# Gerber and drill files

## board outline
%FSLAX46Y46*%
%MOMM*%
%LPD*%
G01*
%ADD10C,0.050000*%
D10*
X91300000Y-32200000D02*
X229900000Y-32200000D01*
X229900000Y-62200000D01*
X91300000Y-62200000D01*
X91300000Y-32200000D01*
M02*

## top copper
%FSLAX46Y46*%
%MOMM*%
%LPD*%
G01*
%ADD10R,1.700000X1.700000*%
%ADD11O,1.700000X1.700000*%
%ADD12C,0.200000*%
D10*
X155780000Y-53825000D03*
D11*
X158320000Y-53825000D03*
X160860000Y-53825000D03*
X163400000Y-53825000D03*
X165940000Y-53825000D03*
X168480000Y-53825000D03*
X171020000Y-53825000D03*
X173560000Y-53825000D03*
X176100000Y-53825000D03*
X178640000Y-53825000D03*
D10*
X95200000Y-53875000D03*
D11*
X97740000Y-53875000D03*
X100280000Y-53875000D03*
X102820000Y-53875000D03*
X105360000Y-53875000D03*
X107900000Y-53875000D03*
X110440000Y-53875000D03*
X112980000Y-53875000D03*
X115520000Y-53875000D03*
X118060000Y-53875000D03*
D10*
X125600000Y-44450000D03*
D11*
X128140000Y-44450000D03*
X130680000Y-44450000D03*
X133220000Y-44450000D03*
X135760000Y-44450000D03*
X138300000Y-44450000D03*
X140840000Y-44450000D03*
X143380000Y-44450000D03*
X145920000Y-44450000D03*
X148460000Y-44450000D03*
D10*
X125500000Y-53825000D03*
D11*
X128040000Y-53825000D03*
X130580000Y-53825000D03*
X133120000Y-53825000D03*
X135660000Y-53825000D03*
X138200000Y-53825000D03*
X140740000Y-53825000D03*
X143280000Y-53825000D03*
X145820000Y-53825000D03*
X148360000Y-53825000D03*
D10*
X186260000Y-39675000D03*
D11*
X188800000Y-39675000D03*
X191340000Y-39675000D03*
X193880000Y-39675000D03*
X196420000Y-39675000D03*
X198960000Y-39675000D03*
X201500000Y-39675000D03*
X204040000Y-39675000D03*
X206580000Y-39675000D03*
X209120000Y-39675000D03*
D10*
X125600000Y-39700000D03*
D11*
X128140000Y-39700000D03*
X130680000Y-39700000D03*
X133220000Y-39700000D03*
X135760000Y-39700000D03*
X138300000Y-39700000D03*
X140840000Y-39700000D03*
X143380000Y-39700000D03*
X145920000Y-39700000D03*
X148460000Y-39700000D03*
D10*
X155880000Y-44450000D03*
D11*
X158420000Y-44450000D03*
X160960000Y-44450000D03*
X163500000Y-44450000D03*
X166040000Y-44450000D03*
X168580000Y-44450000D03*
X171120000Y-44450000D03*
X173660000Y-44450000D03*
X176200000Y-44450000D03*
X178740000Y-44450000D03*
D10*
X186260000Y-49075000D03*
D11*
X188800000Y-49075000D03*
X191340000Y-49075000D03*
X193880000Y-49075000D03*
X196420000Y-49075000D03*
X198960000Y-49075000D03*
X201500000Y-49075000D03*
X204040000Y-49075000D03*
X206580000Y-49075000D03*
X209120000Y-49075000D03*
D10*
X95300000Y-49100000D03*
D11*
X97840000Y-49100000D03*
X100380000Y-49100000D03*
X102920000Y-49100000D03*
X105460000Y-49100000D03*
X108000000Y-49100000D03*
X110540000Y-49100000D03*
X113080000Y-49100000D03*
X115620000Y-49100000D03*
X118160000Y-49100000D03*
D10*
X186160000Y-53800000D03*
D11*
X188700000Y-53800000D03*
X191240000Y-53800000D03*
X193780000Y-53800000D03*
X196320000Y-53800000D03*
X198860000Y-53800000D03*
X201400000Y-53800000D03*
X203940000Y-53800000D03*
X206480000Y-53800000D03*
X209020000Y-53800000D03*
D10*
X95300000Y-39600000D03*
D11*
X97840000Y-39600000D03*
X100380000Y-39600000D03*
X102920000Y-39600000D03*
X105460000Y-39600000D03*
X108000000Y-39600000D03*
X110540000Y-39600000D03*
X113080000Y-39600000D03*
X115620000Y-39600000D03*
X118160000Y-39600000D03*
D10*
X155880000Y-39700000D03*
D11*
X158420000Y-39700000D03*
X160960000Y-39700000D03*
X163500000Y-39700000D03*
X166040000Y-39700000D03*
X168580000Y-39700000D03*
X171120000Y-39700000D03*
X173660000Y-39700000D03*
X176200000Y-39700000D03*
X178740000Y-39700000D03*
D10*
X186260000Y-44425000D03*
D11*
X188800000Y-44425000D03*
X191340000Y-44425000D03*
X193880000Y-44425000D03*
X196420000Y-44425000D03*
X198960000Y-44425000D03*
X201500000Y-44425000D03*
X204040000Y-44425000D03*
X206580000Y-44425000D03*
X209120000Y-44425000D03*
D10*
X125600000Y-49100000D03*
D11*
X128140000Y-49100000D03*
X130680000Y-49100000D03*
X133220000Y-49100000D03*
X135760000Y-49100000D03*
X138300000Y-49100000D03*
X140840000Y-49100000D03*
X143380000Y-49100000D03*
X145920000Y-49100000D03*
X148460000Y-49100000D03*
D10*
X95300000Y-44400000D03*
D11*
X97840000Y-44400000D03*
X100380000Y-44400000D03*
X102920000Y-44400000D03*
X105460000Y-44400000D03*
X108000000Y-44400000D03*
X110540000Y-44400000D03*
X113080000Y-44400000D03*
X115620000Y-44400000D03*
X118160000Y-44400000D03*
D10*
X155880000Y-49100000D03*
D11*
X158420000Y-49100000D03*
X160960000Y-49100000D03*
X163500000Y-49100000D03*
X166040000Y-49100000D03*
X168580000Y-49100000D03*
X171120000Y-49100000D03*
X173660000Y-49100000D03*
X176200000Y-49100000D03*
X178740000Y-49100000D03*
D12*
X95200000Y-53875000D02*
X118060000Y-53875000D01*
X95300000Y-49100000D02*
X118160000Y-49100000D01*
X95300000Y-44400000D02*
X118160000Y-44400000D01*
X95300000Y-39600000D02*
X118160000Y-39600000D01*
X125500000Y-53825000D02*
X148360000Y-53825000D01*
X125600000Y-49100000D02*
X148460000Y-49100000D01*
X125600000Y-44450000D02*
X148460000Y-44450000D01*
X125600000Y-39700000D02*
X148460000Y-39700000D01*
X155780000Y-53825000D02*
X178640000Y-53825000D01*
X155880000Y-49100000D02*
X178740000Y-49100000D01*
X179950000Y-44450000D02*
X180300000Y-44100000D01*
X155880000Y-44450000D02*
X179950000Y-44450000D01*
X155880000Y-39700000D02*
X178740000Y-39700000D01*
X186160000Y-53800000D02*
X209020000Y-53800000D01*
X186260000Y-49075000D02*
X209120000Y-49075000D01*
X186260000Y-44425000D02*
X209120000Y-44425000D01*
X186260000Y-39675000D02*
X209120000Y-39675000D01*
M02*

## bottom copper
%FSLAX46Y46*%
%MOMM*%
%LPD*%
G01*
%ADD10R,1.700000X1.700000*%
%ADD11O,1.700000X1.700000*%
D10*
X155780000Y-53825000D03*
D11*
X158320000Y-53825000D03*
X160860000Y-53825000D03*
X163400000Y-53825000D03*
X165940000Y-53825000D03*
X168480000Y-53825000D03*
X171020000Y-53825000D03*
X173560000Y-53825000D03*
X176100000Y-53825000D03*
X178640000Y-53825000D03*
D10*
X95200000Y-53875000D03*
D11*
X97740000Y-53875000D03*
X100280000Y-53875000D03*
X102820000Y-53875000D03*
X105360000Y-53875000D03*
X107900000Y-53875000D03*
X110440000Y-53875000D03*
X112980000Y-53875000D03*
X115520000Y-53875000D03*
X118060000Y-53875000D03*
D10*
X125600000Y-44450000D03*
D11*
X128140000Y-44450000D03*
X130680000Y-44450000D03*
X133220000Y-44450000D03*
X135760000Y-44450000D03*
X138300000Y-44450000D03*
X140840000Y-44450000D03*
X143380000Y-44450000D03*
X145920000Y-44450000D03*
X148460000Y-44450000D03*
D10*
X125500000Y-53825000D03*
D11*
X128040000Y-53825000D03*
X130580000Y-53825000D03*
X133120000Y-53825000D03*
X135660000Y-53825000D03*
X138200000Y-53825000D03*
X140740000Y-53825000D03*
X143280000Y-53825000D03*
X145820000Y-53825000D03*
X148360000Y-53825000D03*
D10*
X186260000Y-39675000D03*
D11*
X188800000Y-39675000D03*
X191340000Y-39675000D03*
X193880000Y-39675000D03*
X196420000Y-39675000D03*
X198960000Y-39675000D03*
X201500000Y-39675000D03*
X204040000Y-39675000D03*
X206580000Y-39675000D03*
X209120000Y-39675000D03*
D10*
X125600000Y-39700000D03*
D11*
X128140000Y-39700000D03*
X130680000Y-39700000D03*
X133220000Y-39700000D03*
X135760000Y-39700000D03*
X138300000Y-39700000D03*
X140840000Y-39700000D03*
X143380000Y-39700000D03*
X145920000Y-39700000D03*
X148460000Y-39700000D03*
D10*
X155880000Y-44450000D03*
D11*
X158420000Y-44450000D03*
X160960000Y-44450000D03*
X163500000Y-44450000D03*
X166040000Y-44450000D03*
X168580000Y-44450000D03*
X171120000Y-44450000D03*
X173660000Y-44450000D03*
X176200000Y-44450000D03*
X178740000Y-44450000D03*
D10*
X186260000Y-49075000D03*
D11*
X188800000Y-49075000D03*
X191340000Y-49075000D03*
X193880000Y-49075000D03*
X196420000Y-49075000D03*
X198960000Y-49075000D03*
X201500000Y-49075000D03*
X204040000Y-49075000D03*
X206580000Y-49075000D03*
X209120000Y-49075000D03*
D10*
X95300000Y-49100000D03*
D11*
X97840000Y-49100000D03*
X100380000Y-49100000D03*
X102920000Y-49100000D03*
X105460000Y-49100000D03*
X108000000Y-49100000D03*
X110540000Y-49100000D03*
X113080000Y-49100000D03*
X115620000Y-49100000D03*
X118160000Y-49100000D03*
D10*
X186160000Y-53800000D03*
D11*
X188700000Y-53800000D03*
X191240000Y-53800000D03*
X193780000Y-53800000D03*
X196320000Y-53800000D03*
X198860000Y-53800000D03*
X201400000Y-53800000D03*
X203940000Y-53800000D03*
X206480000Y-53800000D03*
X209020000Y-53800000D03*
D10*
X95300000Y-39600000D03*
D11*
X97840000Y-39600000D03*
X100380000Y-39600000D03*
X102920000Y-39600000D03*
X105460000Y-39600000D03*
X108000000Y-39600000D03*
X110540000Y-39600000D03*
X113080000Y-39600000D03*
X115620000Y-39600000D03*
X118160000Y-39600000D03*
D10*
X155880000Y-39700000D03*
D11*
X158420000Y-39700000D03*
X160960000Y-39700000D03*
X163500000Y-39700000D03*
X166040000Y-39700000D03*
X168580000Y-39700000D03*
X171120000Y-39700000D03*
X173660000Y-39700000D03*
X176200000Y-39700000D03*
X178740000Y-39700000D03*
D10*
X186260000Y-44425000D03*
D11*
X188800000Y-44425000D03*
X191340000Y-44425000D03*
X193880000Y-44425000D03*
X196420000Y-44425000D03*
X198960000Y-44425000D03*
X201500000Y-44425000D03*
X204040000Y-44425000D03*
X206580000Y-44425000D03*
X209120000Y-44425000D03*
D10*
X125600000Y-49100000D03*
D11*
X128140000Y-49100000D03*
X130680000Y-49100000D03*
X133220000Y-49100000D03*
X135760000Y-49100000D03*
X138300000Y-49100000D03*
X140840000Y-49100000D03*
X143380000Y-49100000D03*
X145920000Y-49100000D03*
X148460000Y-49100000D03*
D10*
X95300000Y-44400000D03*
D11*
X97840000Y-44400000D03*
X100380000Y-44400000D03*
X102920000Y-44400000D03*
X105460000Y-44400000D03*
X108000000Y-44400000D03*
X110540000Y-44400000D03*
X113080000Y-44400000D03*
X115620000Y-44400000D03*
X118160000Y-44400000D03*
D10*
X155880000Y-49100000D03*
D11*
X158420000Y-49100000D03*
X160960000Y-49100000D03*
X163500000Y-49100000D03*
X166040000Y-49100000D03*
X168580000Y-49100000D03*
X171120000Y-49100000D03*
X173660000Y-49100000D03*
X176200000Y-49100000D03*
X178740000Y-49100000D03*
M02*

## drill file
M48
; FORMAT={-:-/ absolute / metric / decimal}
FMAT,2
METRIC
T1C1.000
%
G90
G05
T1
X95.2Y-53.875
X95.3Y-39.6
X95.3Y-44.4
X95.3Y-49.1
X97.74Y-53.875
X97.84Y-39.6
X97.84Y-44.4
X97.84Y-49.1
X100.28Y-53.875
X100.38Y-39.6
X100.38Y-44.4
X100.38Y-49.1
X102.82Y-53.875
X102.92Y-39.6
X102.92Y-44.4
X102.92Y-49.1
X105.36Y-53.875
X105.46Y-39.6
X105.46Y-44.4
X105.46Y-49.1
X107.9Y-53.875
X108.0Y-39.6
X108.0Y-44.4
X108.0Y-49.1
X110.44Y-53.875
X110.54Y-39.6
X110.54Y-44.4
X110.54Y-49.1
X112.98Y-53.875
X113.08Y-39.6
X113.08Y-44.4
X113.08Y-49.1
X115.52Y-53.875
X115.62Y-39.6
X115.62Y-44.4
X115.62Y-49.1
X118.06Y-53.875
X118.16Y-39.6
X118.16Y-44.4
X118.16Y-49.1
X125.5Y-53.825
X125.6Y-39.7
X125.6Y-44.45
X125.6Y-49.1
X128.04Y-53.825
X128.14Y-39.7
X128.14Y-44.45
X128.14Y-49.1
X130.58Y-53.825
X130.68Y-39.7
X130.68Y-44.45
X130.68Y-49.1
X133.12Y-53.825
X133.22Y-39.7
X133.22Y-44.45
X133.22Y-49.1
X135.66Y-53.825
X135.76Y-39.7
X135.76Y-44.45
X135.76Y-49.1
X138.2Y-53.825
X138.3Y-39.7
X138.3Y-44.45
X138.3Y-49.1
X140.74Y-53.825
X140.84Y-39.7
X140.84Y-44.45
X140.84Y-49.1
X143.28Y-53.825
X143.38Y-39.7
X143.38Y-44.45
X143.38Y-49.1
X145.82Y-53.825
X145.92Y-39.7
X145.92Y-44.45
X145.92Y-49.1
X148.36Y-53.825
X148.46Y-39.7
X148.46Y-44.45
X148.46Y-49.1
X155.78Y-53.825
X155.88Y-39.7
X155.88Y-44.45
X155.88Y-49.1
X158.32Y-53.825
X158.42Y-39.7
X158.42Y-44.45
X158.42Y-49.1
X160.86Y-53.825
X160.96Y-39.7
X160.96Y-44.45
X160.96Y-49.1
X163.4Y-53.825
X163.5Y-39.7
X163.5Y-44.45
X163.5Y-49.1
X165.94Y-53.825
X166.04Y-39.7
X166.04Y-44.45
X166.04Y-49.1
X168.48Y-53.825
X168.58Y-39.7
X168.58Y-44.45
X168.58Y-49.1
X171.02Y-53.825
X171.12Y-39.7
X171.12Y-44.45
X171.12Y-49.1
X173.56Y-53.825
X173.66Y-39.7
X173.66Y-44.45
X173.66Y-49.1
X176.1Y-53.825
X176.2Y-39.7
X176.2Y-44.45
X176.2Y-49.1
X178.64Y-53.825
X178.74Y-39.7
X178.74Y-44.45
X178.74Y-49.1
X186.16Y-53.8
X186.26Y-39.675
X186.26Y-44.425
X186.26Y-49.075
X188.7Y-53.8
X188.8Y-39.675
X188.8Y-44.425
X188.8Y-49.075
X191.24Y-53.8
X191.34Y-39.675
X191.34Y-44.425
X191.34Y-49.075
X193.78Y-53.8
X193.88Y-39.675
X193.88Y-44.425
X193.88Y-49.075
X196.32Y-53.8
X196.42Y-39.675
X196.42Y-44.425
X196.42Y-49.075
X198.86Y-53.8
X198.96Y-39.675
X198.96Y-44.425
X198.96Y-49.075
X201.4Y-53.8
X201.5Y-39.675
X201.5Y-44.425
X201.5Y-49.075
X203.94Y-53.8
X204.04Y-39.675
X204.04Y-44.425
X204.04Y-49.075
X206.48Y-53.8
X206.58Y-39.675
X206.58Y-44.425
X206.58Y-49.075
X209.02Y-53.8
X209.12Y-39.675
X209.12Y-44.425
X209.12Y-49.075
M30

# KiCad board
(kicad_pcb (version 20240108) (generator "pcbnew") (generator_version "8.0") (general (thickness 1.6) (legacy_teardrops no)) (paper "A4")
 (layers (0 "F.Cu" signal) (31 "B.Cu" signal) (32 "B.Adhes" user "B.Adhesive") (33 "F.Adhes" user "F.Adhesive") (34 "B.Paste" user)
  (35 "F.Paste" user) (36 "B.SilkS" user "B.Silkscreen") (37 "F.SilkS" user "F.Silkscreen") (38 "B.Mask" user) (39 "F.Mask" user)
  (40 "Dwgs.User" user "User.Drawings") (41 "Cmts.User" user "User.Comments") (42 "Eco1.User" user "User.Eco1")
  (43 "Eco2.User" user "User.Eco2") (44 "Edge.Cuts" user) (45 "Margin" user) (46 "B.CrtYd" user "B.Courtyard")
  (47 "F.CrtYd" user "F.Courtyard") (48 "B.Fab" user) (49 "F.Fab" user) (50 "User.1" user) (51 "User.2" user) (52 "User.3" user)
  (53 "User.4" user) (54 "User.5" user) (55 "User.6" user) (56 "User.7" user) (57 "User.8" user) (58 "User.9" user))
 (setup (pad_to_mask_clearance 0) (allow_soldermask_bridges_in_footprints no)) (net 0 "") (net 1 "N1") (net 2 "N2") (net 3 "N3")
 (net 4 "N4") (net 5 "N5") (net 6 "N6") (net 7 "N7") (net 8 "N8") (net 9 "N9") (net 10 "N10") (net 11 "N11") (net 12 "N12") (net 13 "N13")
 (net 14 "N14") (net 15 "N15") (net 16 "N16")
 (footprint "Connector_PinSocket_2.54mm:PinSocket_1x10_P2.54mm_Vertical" (layer "F.Cu") (at 155.78 53.825 90)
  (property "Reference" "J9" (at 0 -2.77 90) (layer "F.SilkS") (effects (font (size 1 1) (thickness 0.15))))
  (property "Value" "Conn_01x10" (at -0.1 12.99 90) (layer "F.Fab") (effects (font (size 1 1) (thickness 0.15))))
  (pad "1" thru_hole rect (at 0 0 90) (size 1.7 1.7) (drill 1) (layers "*.Cu" "*.Mask") (remove_unused_layers no) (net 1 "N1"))
  (pad "2" thru_hole oval (at 0 2.54 90) (size 1.7 1.7) (drill 1) (layers "*.Cu" "*.Mask") (remove_unused_layers no) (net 1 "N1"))
  (pad "3" thru_hole oval (at 0 5.08 90) (size 1.7 1.7) (drill 1) (layers "*.Cu" "*.Mask") (remove_unused_layers no) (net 1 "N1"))
  (pad "4" thru_hole oval (at 0 7.62 90) (size 1.7 1.7) (drill 1) (layers "*.Cu" "*.Mask") (remove_unused_layers no) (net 1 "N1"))
  (pad "5" thru_hole oval (at 0 10.16 90) (size 1.7 1.7) (drill 1) (layers "*.Cu" "*.Mask") (remove_unused_layers no) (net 1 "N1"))
  (pad "6" thru_hole oval (at 0 12.7 90) (size 1.7 1.7) (drill 1) (layers "*.Cu" "*.Mask") (remove_unused_layers no) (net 1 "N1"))
  (pad "7" thru_hole oval (at 0 15.24 90) (size 1.7 1.7) (drill 1) (layers "*.Cu" "*.Mask") (remove_unused_layers no) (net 1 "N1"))
  (pad "8" thru_hole oval (at 0 17.78 90) (size 1.7 1.7) (drill 1) (layers "*.Cu" "*.Mask") (remove_unused_layers no) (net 1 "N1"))
  (pad "9" thru_hole oval (at 0 20.32 90) (size 1.7 1.7) (drill 1) (layers "*.Cu" "*.Mask") (remove_unused_layers no) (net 1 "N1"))
  (pad "10" thru_hole oval (at 0 22.86 90) (size 1.7 1.7) (drill 1) (layers "*.Cu" "*.Mask") (remove_unused_layers no) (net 1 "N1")))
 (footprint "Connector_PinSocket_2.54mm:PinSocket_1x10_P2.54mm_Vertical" (layer "F.Cu") (at 95.2 53.875 90)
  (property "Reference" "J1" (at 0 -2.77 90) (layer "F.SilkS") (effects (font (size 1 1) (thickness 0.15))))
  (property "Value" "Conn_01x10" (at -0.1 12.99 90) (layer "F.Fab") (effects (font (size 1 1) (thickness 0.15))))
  (pad "1" thru_hole rect (at 0 0 90) (size 1.7 1.7) (drill 1) (layers "*.Cu" "*.Mask") (remove_unused_layers no) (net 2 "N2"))
  (pad "2" thru_hole oval (at 0 2.54 90) (size 1.7 1.7) (drill 1) (layers "*.Cu" "*.Mask") (remove_unused_layers no) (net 2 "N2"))
  (pad "3" thru_hole oval (at 0 5.08 90) (size 1.7 1.7) (drill 1) (layers "*.Cu" "*.Mask") (remove_unused_layers no) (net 2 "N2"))
  (pad "4" thru_hole oval (at 0 7.62 90) (size 1.7 1.7) (drill 1) (layers "*.Cu" "*.Mask") (remove_unused_layers no) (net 2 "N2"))
  (pad "5" thru_hole oval (at 0 10.16 90) (size 1.7 1.7) (drill 1) (layers "*.Cu" "*.Mask") (remove_unused_layers no) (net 2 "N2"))
  (pad "6" thru_hole oval (at 0 12.7 90) (size 1.7 1.7) (drill 1) (layers "*.Cu" "*.Mask") (remove_unused_layers no) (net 2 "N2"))
  (pad "7" thru_hole oval (at 0 15.24 90) (size 1.7 1.7) (drill 1) (layers "*.Cu" "*.Mask") (remove_unused_layers no) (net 2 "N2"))
  (pad "8" thru_hole oval (at 0 17.78 90) (size 1.7 1.7) (drill 1) (layers "*.Cu" "*.Mask") (remove_unused_layers no) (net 2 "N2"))
  (pad "9" thru_hole oval (at 0 20.32 90) (size 1.7 1.7) (drill 1) (layers "*.Cu" "*.Mask") (remove_unused_layers no) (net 2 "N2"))
  (pad "10" thru_hole oval (at 0 22.86 90) (size 1.7 1.7) (drill 1) (layers "*.Cu" "*.Mask") (remove_unused_layers no) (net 2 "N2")))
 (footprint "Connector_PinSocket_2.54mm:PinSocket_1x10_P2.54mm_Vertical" (layer "F.Cu") (at 125.6 44.45 90)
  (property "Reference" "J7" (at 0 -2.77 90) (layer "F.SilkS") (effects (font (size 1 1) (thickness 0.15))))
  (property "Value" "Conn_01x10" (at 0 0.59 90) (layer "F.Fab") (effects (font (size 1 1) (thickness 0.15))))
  (pad "1" thru_hole rect (at 0 0 90) (size 1.7 1.7) (drill 1) (layers "*.Cu" "*.Mask") (remove_unused_layers no) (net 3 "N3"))
  (pad "2" thru_hole oval (at 0 2.54 90) (size 1.7 1.7) (drill 1) (layers "*.Cu" "*.Mask") (remove_unused_layers no) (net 3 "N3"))
  (pad "3" thru_hole oval (at 0 5.08 90) (size 1.7 1.7) (drill 1) (layers "*.Cu" "*.Mask") (remove_unused_layers no) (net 3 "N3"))
  (pad "4" thru_hole oval (at 0 7.62 90) (size 1.7 1.7) (drill 1) (layers "*.Cu" "*.Mask") (remove_unused_layers no) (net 3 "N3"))
  (pad "5" thru_hole oval (at 0 10.16 90) (size 1.7 1.7) (drill 1) (layers "*.Cu" "*.Mask") (remove_unused_layers no) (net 3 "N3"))
  (pad "6" thru_hole oval (at 0 12.7 90) (size 1.7 1.7) (drill 1) (layers "*.Cu" "*.Mask") (remove_unused_layers no) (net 3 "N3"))
  (pad "7" thru_hole oval (at 0 15.24 90) (size 1.7 1.7) (drill 1) (layers "*.Cu" "*.Mask") (remove_unused_layers no) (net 3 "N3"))
  (pad "8" thru_hole oval (at 0 17.78 90) (size 1.7 1.7) (drill 1) (layers "*.Cu" "*.Mask") (remove_unused_layers no) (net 3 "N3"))
  (pad "9" thru_hole oval (at 0 20.32 90) (size 1.7 1.7) (drill 1) (layers "*.Cu" "*.Mask") (remove_unused_layers no) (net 3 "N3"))
  (pad "10" thru_hole oval (at 0 22.86 90) (size 1.7 1.7) (drill 1) (layers "*.Cu" "*.Mask") (remove_unused_layers no) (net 3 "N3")))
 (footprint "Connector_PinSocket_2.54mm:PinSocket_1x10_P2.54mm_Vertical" (layer "F.Cu") (at 125.5 53.825 90)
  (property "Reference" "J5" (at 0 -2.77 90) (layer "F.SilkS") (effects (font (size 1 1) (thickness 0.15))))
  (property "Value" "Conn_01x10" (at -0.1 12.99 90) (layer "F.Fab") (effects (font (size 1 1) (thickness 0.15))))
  (pad "1" thru_hole rect (at 0 0 90) (size 1.7 1.7) (drill 1) (layers "*.Cu" "*.Mask") (remove_unused_layers no) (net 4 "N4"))
  (pad "2" thru_hole oval (at 0 2.54 90) (size 1.7 1.7) (drill 1) (layers "*.Cu" "*.Mask") (remove_unused_layers no) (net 4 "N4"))
  (pad "3" thru_hole oval (at 0 5.08 90) (size 1.7 1.7) (drill 1) (layers "*.Cu" "*.Mask") (remove_unused_layers no) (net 4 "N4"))
  (pad "4" thru_hole oval (at 0 7.62 90) (size 1.7 1.7) (drill 1) (layers "*.Cu" "*.Mask") (remove_unused_layers no) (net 4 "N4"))
  (pad "5" thru_hole oval (at 0 10.16 90) (size 1.7 1.7) (drill 1) (layers "*.Cu" "*.Mask") (remove_unused_layers no) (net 4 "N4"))
  (pad "6" thru_hole oval (at 0 12.7 90) (size 1.7 1.7) (drill 1) (layers "*.Cu" "*.Mask") (remove_unused_layers no) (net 4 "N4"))
  (pad "7" thru_hole oval (at 0 15.24 90) (size 1.7 1.7) (drill 1) (layers "*.Cu" "*.Mask") (remove_unused_layers no) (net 4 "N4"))
  (pad "8" thru_hole oval (at 0 17.78 90) (size 1.7 1.7) (drill 1) (layers "*.Cu" "*.Mask") (remove_unused_layers no) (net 4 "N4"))
  (pad "9" thru_hole oval (at 0 20.32 90) (size 1.7 1.7) (drill 1) (layers "*.Cu" "*.Mask") (remove_unused_layers no) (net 4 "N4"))
  (pad "10" thru_hole oval (at 0 22.86 90) (size 1.7 1.7) (drill 1) (layers "*.Cu" "*.Mask") (remove_unused_layers no) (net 4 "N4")))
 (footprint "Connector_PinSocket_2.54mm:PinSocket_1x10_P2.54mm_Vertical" (layer "F.Cu") (at 186.26 39.675 90)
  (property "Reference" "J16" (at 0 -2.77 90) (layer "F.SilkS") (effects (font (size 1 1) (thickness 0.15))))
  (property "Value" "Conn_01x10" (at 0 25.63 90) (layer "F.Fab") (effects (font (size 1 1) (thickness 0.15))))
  (pad "1" thru_hole rect (at 0 0 90) (size 1.7 1.7) (drill 1) (layers "*.Cu" "*.Mask") (remove_unused_layers no) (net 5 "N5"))
  (pad "2" thru_hole oval (at 0 2.54 90) (size 1.7 1.7) (drill 1) (layers "*.Cu" "*.Mask") (remove_unused_layers no) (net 5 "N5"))
  (pad "3" thru_hole oval (at 0 5.08 90) (size 1.7 1.7) (drill 1) (layers "*.Cu" "*.Mask") (remove_unused_layers no) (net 5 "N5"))
  (pad "4" thru_hole oval (at 0 7.62 90) (size 1.7 1.7) (drill 1) (layers "*.Cu" "*.Mask") (remove_unused_layers no) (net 5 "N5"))
  (pad "5" thru_hole oval (at 0 10.16 90) (size 1.7 1.7) (drill 1) (layers "*.Cu" "*.Mask") (remove_unused_layers no) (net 5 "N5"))
  (pad "6" thru_hole oval (at 0 12.7 90) (size 1.7 1.7) (drill 1) (layers "*.Cu" "*.Mask") (remove_unused_layers no) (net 5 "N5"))
  (pad "7" thru_hole oval (at 0 15.24 90) (size 1.7 1.7) (drill 1) (layers "*.Cu" "*.Mask") (remove_unused_layers no) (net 5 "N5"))
  (pad "8" thru_hole oval (at 0 17.78 90) (size 1.7 1.7) (drill 1) (layers "*.Cu" "*.Mask") (remove_unused_layers no) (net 5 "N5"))
  (pad "9" thru_hole oval (at 0 20.32 90) (size 1.7 1.7) (drill 1) (layers "*.Cu" "*.Mask") (remove_unused_layers no) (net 5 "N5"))
  (pad "10" thru_hole oval (at 0 22.86 90) (size 1.7 1.7) (drill 1) (layers "*.Cu" "*.Mask") (remove_unused_layers no) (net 5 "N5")))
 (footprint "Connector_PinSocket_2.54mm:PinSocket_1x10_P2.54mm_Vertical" (layer "F.Cu") (at 125.6 39.7 90)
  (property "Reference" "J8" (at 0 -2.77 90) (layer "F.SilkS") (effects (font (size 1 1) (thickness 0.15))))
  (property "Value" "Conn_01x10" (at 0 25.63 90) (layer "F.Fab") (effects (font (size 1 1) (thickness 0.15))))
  (pad "1" thru_hole rect (at 0 0 90) (size 1.7 1.7) (drill 1) (layers "*.Cu" "*.Mask") (remove_unused_layers no) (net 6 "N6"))
  (pad "2" thru_hole oval (at 0 2.54 90) (size 1.7 1.7) (drill 1) (layers "*.Cu" "*.Mask") (remove_unused_layers no) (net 6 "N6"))
  (pad "3" thru_hole oval (at 0 5.08 90) (size 1.7 1.7) (drill 1) (layers "*.Cu" "*.Mask") (remove_unused_layers no) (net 6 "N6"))
  (pad "4" thru_hole oval (at 0 7.62 90) (size 1.7 1.7) (drill 1) (layers "*.Cu" "*.Mask") (remove_unused_layers no) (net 6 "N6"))
  (pad "5" thru_hole oval (at 0 10.16 90) (size 1.7 1.7) (drill 1) (layers "*.Cu" "*.Mask") (remove_unused_layers no) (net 6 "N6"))
  (pad "6" thru_hole oval (at 0 12.7 90) (size 1.7 1.7) (drill 1) (layers "*.Cu" "*.Mask") (remove_unused_layers no) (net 6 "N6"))
  (pad "7" thru_hole oval (at 0 15.24 90) (size 1.7 1.7) (drill 1) (layers "*.Cu" "*.Mask") (remove_unused_layers no) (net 6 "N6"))
  (pad "8" thru_hole oval (at 0 17.78 90) (size 1.7 1.7) (drill 1) (layers "*.Cu" "*.Mask") (remove_unused_layers no) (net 6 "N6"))
  (pad "9" thru_hole oval (at 0 20.32 90) (size 1.7 1.7) (drill 1) (layers "*.Cu" "*.Mask") (remove_unused_layers no) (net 6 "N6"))
  (pad "10" thru_hole oval (at 0 22.86 90) (size 1.7 1.7) (drill 1) (layers "*.Cu" "*.Mask") (remove_unused_layers no) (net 6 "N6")))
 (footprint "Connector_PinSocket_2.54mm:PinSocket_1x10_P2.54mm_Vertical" (layer "F.Cu") (at 155.88 44.45 90)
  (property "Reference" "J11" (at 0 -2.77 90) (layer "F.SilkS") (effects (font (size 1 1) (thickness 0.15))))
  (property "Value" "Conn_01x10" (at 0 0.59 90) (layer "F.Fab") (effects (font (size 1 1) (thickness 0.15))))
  (pad "1" thru_hole rect (at 0 0 90) (size 1.7 1.7) (drill 1) (layers "*.Cu" "*.Mask") (remove_unused_layers no) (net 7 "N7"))
  (pad "2" thru_hole oval (at 0 2.54 90) (size 1.7 1.7) (drill 1) (layers "*.Cu" "*.Mask") (remove_unused_layers no) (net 7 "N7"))
  (pad "3" thru_hole oval (at 0 5.08 90) (size 1.7 1.7) (drill 1) (layers "*.Cu" "*.Mask") (remove_unused_layers no) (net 7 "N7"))
  (pad "4" thru_hole oval (at 0 7.62 90) (size 1.7 1.7) (drill 1) (layers "*.Cu" "*.Mask") (remove_unused_layers no) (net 7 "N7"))
  (pad "5" thru_hole oval (at 0 10.16 90) (size 1.7 1.7) (drill 1) (layers "*.Cu" "*.Mask") (remove_unused_layers no) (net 7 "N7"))
  (pad "6" thru_hole oval (at 0 12.7 90) (size 1.7 1.7) (drill 1) (layers "*.Cu" "*.Mask") (remove_unused_layers no) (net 7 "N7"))
  (pad "7" thru_hole oval (at 0 15.24 90) (size 1.7 1.7) (drill 1) (layers "*.Cu" "*.Mask") (remove_unused_layers no) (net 7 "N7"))
  (pad "8" thru_hole oval (at 0 17.78 90) (size 1.7 1.7) (drill 1) (layers "*.Cu" "*.Mask") (remove_unused_layers no) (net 7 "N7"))
  (pad "9" thru_hole oval (at 0 20.32 90) (size 1.7 1.7) (drill 1) (layers "*.Cu" "*.Mask") (remove_unused_layers no) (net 7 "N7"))
  (pad "10" thru_hole oval (at 0 22.86 90) (size 1.7 1.7) (drill 1) (layers "*.Cu" "*.Mask") (remove_unused_layers no) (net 7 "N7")))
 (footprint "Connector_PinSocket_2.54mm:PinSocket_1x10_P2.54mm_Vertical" (layer "F.Cu") (at 186.26 49.075 90)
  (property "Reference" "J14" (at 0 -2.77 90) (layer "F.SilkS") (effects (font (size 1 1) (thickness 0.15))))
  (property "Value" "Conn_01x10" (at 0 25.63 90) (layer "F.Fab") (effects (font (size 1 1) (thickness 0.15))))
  (pad "1" thru_hole rect (at 0 0 90) (size 1.7 1.7) (drill 1) (layers "*.Cu" "*.Mask") (remove_unused_layers no) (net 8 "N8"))
  (pad "2" thru_hole oval (at 0 2.54 90) (size 1.7 1.7) (drill 1) (layers "*.Cu" "*.Mask") (remove_unused_layers no) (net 8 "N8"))
  (pad "3" thru_hole oval (at 0 5.08 90) (size 1.7 1.7) (drill 1) (layers "*.Cu" "*.Mask") (remove_unused_layers no) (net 8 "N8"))
  (pad "4" thru_hole oval (at 0 7.62 90) (size 1.7 1.7) (drill 1) (layers "*.Cu" "*.Mask") (remove_unused_layers no) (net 8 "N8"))
  (pad "5" thru_hole oval (at 0 10.16 90) (size 1.7 1.7) (drill 1) (layers "*.Cu" "*.Mask") (remove_unused_layers no) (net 8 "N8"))
  (pad "6" thru_hole oval (at 0 12.7 90) (size 1.7 1.7) (drill 1) (layers "*.Cu" "*.Mask") (remove_unused_layers no) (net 8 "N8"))
  (pad "7" thru_hole oval (at 0 15.24 90) (size 1.7 1.7) (drill 1) (layers "*.Cu" "*.Mask") (remove_unused_layers no) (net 8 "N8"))
  (pad "8" thru_hole oval (at 0 17.78 90) (size 1.7 1.7) (drill 1) (layers "*.Cu" "*.Mask") (remove_unused_layers no) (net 8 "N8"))
  (pad "9" thru_hole oval (at 0 20.32 90) (size 1.7 1.7) (drill 1) (layers "*.Cu" "*.Mask") (remove_unused_layers no) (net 8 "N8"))
  (pad "10" thru_hole oval (at 0 22.86 90) (size 1.7 1.7) (drill 1) (layers "*.Cu" "*.Mask") (remove_unused_layers no) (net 8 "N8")))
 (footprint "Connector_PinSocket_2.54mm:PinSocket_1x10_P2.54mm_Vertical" (layer "F.Cu") (at 95.3 49.1 90)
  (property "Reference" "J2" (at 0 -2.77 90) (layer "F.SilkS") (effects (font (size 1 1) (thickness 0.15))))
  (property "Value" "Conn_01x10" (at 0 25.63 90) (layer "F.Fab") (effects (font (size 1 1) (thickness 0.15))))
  (pad "1" thru_hole rect (at 0 0 90) (size 1.7 1.7) (drill 1) (layers "*.Cu" "*.Mask") (remove_unused_layers no) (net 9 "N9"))
  (pad "2" thru_hole oval (at 0 2.54 90) (size 1.7 1.7) (drill 1) (layers "*.Cu" "*.Mask") (remove_unused_layers no) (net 9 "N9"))
  (pad "3" thru_hole oval (at 0 5.08 90) (size 1.7 1.7) (drill 1) (layers "*.Cu" "*.Mask") (remove_unused_layers no) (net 9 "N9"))
  (pad "4" thru_hole oval (at 0 7.62 90) (size 1.7 1.7) (drill 1) (layers "*.Cu" "*.Mask") (remove_unused_layers no) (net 9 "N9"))
  (pad "5" thru_hole oval (at 0 10.16 90) (size 1.7 1.7) (drill 1) (layers "*.Cu" "*.Mask") (remove_unused_layers no) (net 9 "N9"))
  (pad "6" thru_hole oval (at 0 12.7 90) (size 1.7 1.7) (drill 1) (layers "*.Cu" "*.Mask") (remove_unused_layers no) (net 9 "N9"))
  (pad "7" thru_hole oval (at 0 15.24 90) (size 1.7 1.7) (drill 1) (layers "*.Cu" "*.Mask") (remove_unused_layers no) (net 9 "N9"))
  (pad "8" thru_hole oval (at 0 17.78 90) (size 1.7 1.7) (drill 1) (layers "*.Cu" "*.Mask") (remove_unused_layers no) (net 9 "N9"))
  (pad "9" thru_hole oval (at 0 20.32 90) (size 1.7 1.7) (drill 1) (layers "*.Cu" "*.Mask") (remove_unused_layers no) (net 9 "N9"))
  (pad "10" thru_hole oval (at 0 22.86 90) (size 1.7 1.7) (drill 1) (layers "*.Cu" "*.Mask") (remove_unused_layers no) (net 9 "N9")))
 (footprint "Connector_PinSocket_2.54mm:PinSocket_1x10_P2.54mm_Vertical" (layer "F.Cu") (at 186.16 53.8 90)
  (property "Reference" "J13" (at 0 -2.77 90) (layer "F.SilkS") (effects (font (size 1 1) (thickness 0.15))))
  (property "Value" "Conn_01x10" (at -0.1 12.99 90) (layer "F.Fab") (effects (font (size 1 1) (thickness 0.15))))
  (pad "1" thru_hole rect (at 0 0 90) (size 1.7 1.7) (drill 1) (layers "*.Cu" "*.Mask") (remove_unused_layers no) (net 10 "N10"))
  (pad "2" thru_hole oval (at 0 2.54 90) (size 1.7 1.7) (drill 1) (layers "*.Cu" "*.Mask") (remove_unused_layers no) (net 10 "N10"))
  (pad "3" thru_hole oval (at 0 5.08 90) (size 1.7 1.7) (drill 1) (layers "*.Cu" "*.Mask") (remove_unused_layers no) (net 10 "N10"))
  (pad "4" thru_hole oval (at 0 7.62 90) (size 1.7 1.7) (drill 1) (layers "*.Cu" "*.Mask") (remove_unused_layers no) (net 10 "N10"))
  (pad "5" thru_hole oval (at 0 10.16 90) (size 1.7 1.7) (drill 1) (layers "*.Cu" "*.Mask") (remove_unused_layers no) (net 10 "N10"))
  (pad "6" thru_hole oval (at 0 12.7 90) (size 1.7 1.7) (drill 1) (layers "*.Cu" "*.Mask") (remove_unused_layers no) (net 10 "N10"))
  (pad "7" thru_hole oval (at 0 15.24 90) (size 1.7 1.7) (drill 1) (layers "*.Cu" "*.Mask") (remove_unused_layers no) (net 10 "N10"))
  (pad "8" thru_hole oval (at 0 17.78 90) (size 1.7 1.7) (drill 1) (layers "*.Cu" "*.Mask") (remove_unused_layers no) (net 10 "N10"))
  (pad "9" thru_hole oval (at 0 20.32 90) (size 1.7 1.7) (drill 1) (layers "*.Cu" "*.Mask") (remove_unused_layers no) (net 10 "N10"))
  (pad "10" thru_hole oval (at 0 22.86 90) (size 1.7 1.7) (drill 1) (layers "*.Cu" "*.Mask") (remove_unused_layers no) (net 10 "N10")))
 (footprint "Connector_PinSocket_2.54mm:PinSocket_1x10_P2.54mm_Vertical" (layer "F.Cu") (at 95.3 39.6 90)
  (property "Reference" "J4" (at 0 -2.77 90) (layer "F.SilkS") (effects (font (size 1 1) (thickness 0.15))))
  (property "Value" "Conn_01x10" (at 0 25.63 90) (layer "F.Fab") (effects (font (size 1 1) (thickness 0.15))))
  (pad "1" thru_hole rect (at 0 0 90) (size 1.7 1.7) (drill 1) (layers "*.Cu" "*.Mask") (remove_unused_layers no) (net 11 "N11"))
  (pad "2" thru_hole oval (at 0 2.54 90) (size 1.7 1.7) (drill 1) (layers "*.Cu" "*.Mask") (remove_unused_layers no) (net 11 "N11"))
  (pad "3" thru_hole oval (at 0 5.08 90) (size 1.7 1.7) (drill 1) (layers "*.Cu" "*.Mask") (remove_unused_layers no) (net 11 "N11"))
  (pad "4" thru_hole oval (at 0 7.62 90) (size 1.7 1.7) (drill 1) (layers "*.Cu" "*.Mask") (remove_unused_layers no) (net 11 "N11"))
  (pad "5" thru_hole oval (at 0 10.16 90) (size 1.7 1.7) (drill 1) (layers "*.Cu" "*.Mask") (remove_unused_layers no) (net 11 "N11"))
  (pad "6" thru_hole oval (at 0 12.7 90) (size 1.7 1.7) (drill 1) (layers "*.Cu" "*.Mask") (remove_unused_layers no) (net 11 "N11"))
  (pad "7" thru_hole oval (at 0 15.24 90) (size 1.7 1.7) (drill 1) (layers "*.Cu" "*.Mask") (remove_unused_layers no) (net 11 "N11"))
  (pad "8" thru_hole oval (at 0 17.78 90) (size 1.7 1.7) (drill 1) (layers "*.Cu" "*.Mask") (remove_unused_layers no) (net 11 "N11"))
  (pad "9" thru_hole oval (at 0 20.32 90) (size 1.7 1.7) (drill 1) (layers "*.Cu" "*.Mask") (remove_unused_layers no) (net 11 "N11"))
  (pad "10" thru_hole oval (at 0 22.86 90) (size 1.7 1.7) (drill 1) (layers "*.Cu" "*.Mask") (remove_unused_layers no) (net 11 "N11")))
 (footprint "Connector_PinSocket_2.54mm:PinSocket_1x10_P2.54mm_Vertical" (layer "F.Cu") (at 155.88 39.7 90)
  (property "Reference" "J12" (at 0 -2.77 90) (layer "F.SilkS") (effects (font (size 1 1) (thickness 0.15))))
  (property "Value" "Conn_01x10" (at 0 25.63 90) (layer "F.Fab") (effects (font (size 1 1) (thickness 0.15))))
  (pad "1" thru_hole rect (at 0 0 90) (size 1.7 1.7) (drill 1) (layers "*.Cu" "*.Mask") (remove_unused_layers no) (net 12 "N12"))
  (pad "2" thru_hole oval (at 0 2.54 90) (size 1.7 1.7) (drill 1) (layers "*.Cu" "*.Mask") (remove_unused_layers no) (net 12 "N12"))
  (pad "3" thru_hole oval (at 0 5.08 90) (size 1.7 1.7) (drill 1) (layers "*.Cu" "*.Mask") (remove_unused_layers no) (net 12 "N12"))
  (pad "4" thru_hole oval (at 0 7.62 90) (size 1.7 1.7) (drill 1) (layers "*.Cu" "*.Mask") (remove_unused_layers no) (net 12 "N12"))
  (pad "5" thru_hole oval (at 0 10.16 90) (size 1.7 1.7) (drill 1) (layers "*.Cu" "*.Mask") (remove_unused_layers no) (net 12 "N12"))
  (pad "6" thru_hole oval (at 0 12.7 90) (size 1.7 1.7) (drill 1) (layers "*.Cu" "*.Mask") (remove_unused_layers no) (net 12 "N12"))
  (pad "7" thru_hole oval (at 0 15.24 90) (size 1.7 1.7) (drill 1) (layers "*.Cu" "*.Mask") (remove_unused_layers no) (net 12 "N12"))
  (pad "8" thru_hole oval (at 0 17.78 90) (size 1.7 1.7) (drill 1) (layers "*.Cu" "*.Mask") (remove_unused_layers no) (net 12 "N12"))
  (pad "9" thru_hole oval (at 0 20.32 90) (size 1.7 1.7) (drill 1) (layers "*.Cu" "*.Mask") (remove_unused_layers no) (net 12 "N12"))
  (pad "10" thru_hole oval (at 0 22.86 90) (size 1.7 1.7) (drill 1) (layers "*.Cu" "*.Mask") (remove_unused_layers no) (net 12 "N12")))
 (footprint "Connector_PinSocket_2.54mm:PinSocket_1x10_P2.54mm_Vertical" (layer "F.Cu") (at 186.26 44.425 90)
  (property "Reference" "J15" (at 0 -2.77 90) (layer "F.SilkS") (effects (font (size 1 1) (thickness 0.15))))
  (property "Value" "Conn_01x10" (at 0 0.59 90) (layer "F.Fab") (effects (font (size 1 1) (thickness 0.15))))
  (pad "1" thru_hole rect (at 0 0 90) (size 1.7 1.7) (drill 1) (layers "*.Cu" "*.Mask") (remove_unused_layers no) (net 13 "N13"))
  (pad "2" thru_hole oval (at 0 2.54 90) (size 1.7 1.7) (drill 1) (layers "*.Cu" "*.Mask") (remove_unused_layers no) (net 13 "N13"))
  (pad "3" thru_hole oval (at 0 5.08 90) (size 1.7 1.7) (drill 1) (layers "*.Cu" "*.Mask") (remove_unused_layers no) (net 13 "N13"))
  (pad "4" thru_hole oval (at 0 7.62 90) (size 1.7 1.7) (drill 1) (layers "*.Cu" "*.Mask") (remove_unused_layers no) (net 13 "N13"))
  (pad "5" thru_hole oval (at 0 10.16 90) (size 1.7 1.7) (drill 1) (layers "*.Cu" "*.Mask") (remove_unused_layers no) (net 13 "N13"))
  (pad "6" thru_hole oval (at 0 12.7 90) (size 1.7 1.7) (drill 1) (layers "*.Cu" "*.Mask") (remove_unused_layers no) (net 13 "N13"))
  (pad "7" thru_hole oval (at 0 15.24 90) (size 1.7 1.7) (drill 1) (layers "*.Cu" "*.Mask") (remove_unused_layers no) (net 13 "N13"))
  (pad "8" thru_hole oval (at 0 17.78 90) (size 1.7 1.7) (drill 1) (layers "*.Cu" "*.Mask") (remove_unused_layers no) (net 13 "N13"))
  (pad "9" thru_hole oval (at 0 20.32 90) (size 1.7 1.7) (drill 1) (layers "*.Cu" "*.Mask") (remove_unused_layers no) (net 13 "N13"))
  (pad "10" thru_hole oval (at 0 22.86 90) (size 1.7 1.7) (drill 1) (layers "*.Cu" "*.Mask") (remove_unused_layers no) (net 13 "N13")))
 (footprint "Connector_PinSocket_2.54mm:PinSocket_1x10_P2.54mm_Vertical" (layer "F.Cu") (at 125.6 49.1 90)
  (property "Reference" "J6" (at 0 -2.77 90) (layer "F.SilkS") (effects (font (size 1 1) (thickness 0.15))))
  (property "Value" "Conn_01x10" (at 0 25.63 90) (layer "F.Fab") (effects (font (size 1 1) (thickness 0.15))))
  (pad "1" thru_hole rect (at 0 0 90) (size 1.7 1.7) (drill 1) (layers "*.Cu" "*.Mask") (remove_unused_layers no) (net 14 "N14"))
  (pad "2" thru_hole oval (at 0 2.54 90) (size 1.7 1.7) (drill 1) (layers "*.Cu" "*.Mask") (remove_unused_layers no) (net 14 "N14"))
  (pad "3" thru_hole oval (at 0 5.08 90) (size 1.7 1.7) (drill 1) (layers "*.Cu" "*.Mask") (remove_unused_layers no) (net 14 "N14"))
  (pad "4" thru_hole oval (at 0 7.62 90) (size 1.7 1.7) (drill 1) (layers "*.Cu" "*.Mask") (remove_unused_layers no) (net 14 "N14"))
  (pad "5" thru_hole oval (at 0 10.16 90) (size 1.7 1.7) (drill 1) (layers "*.Cu" "*.Mask") (remove_unused_layers no) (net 14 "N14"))
  (pad "6" thru_hole oval (at 0 12.7 90) (size 1.7 1.7) (drill 1) (layers "*.Cu" "*.Mask") (remove_unused_layers no) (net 14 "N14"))
  (pad "7" thru_hole oval (at 0 15.24 90) (size 1.7 1.7) (drill 1) (layers "*.Cu" "*.Mask") (remove_unused_layers no) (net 14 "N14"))
  (pad "8" thru_hole oval (at 0 17.78 90) (size 1.7 1.7) (drill 1) (layers "*.Cu" "*.Mask") (remove_unused_layers no) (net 14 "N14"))
  (pad "9" thru_hole oval (at 0 20.32 90) (size 1.7 1.7) (drill 1) (layers "*.Cu" "*.Mask") (remove_unused_layers no) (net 14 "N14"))
  (pad "10" thru_hole oval (at 0 22.86 90) (size 1.7 1.7) (drill 1) (layers "*.Cu" "*.Mask") (remove_unused_layers no) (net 14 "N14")))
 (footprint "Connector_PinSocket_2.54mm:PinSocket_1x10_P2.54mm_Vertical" (layer "F.Cu") (at 95.3 44.4 90)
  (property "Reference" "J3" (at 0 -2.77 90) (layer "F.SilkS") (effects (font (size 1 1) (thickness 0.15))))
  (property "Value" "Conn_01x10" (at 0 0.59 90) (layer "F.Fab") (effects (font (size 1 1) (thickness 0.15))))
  (pad "1" thru_hole rect (at 0 0 90) (size 1.7 1.7) (drill 1) (layers "*.Cu" "*.Mask") (remove_unused_layers no) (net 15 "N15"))
  (pad "2" thru_hole oval (at 0 2.54 90) (size 1.7 1.7) (drill 1) (layers "*.Cu" "*.Mask") (remove_unused_layers no) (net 15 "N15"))
  (pad "3" thru_hole oval (at 0 5.08 90) (size 1.7 1.7) (drill 1) (layers "*.Cu" "*.Mask") (remove_unused_layers no) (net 15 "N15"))
  (pad "4" thru_hole oval (at 0 7.62 90) (size 1.7 1.7) (drill 1) (layers "*.Cu" "*.Mask") (remove_unused_layers no) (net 15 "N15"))
  (pad "5" thru_hole oval (at 0 10.16 90) (size 1.7 1.7) (drill 1) (layers "*.Cu" "*.Mask") (remove_unused_layers no) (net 15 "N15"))
  (pad "6" thru_hole oval (at 0 12.7 90) (size 1.7 1.7) (drill 1) (layers "*.Cu" "*.Mask") (remove_unused_layers no) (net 15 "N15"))
  (pad "7" thru_hole oval (at 0 15.24 90) (size 1.7 1.7) (drill 1) (layers "*.Cu" "*.Mask") (remove_unused_layers no) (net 15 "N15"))
  (pad "8" thru_hole oval (at 0 17.78 90) (size 1.7 1.7) (drill 1) (layers "*.Cu" "*.Mask") (remove_unused_layers no) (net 15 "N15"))
  (pad "9" thru_hole oval (at 0 20.32 90) (size 1.7 1.7) (drill 1) (layers "*.Cu" "*.Mask") (remove_unused_layers no) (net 15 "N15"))
  (pad "10" thru_hole oval (at 0 22.86 90) (size 1.7 1.7) (drill 1) (layers "*.Cu" "*.Mask") (remove_unused_layers no) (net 15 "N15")))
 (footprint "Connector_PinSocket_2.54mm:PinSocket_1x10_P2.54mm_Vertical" (layer "F.Cu") (at 155.88 49.1 90)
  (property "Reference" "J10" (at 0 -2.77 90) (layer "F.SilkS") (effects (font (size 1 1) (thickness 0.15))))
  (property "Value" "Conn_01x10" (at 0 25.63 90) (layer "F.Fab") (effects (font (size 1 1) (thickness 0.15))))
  (pad "1" thru_hole rect (at 0 0 90) (size 1.7 1.7) (drill 1) (layers "*.Cu" "*.Mask") (remove_unused_layers no) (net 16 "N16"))
  (pad "2" thru_hole oval (at 0 2.54 90) (size 1.7 1.7) (drill 1) (layers "*.Cu" "*.Mask") (remove_unused_layers no) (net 16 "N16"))
  (pad "3" thru_hole oval (at 0 5.08 90) (size 1.7 1.7) (drill 1) (layers "*.Cu" "*.Mask") (remove_unused_layers no) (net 16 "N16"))
  (pad "4" thru_hole oval (at 0 7.62 90) (size 1.7 1.7) (drill 1) (layers "*.Cu" "*.Mask") (remove_unused_layers no) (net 16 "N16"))
  (pad "5" thru_hole oval (at 0 10.16 90) (size 1.7 1.7) (drill 1) (layers "*.Cu" "*.Mask") (remove_unused_layers no) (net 16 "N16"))
  (pad "6" thru_hole oval (at 0 12.7 90) (size 1.7 1.7) (drill 1) (layers "*.Cu" "*.Mask") (remove_unused_layers no) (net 16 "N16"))
  (pad "7" thru_hole oval (at 0 15.24 90) (size 1.7 1.7) (drill 1) (layers "*.Cu" "*.Mask") (remove_unused_layers no) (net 16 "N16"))
  (pad "8" thru_hole oval (at 0 17.78 90) (size 1.7 1.7) (drill 1) (layers "*.Cu" "*.Mask") (remove_unused_layers no) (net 16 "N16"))
  (pad "9" thru_hole oval (at 0 20.32 90) (size 1.7 1.7) (drill 1) (layers "*.Cu" "*.Mask") (remove_unused_layers no) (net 16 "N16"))
  (pad "10" thru_hole oval (at 0 22.86 90) (size 1.7 1.7) (drill 1) (layers "*.Cu" "*.Mask") (remove_unused_layers no) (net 16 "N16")))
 (gr_rect (start 91.3 32.2) (end 229.9 62.2) (stroke (width 0.05) (type default)) (fill none) (layer "Edge.Cuts"))
 (segment (start 95.2 53.875) (end 118.06 53.875) (width 0.2) (layer "F.Cu") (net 2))
 (segment (start 95.3 49.1) (end 118.16 49.1) (width 0.2) (layer "F.Cu") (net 9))
 (segment (start 95.3 44.4) (end 118.16 44.4) (width 0.2) (layer "F.Cu") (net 15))
 (segment (start 95.3 39.6) (end 118.16 39.6) (width 0.2) (layer "F.Cu") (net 11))
 (segment (start 125.5 53.825) (end 148.36 53.825) (width 0.2) (layer "F.Cu") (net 4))
 (segment (start 125.6 49.1) (end 148.46 49.1) (width 0.2) (layer "F.Cu") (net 14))
 (segment (start 125.6 44.45) (end 148.46 44.45) (width 0.2) (layer "F.Cu") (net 3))
 (segment (start 125.6 39.7) (end 148.46 39.7) (width 0.2) (layer "F.Cu") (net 6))
 (segment (start 155.78 53.825) (end 178.64 53.825) (width 0.2) (layer "F.Cu") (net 1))
 (segment (start 155.88 49.1) (end 178.74 49.1) (width 0.2) (layer "F.Cu") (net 16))
 (segment (start 179.95 44.45) (end 180.3 44.1) (width 0.2) (layer "F.Cu") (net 7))
 (segment (start 155.88 44.45) (end 179.95 44.45) (width 0.2) (layer "F.Cu") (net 7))
 (segment (start 155.88 39.7) (end 178.74 39.7) (width 0.2) (layer "F.Cu") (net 12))
 (segment (start 186.16 53.8) (end 209.02 53.8) (width 0.2) (layer "F.Cu") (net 10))
 (segment (start 186.26 49.075) (end 209.12 49.075) (width 0.2) (layer "F.Cu") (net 8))
 (segment (start 186.26 44.425) (end 209.12 44.425) (width 0.2) (layer "F.Cu") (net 13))
 (segment (start 186.26 39.675) (end 209.12 39.675) (width 0.2) (layer "F.Cu") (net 5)))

